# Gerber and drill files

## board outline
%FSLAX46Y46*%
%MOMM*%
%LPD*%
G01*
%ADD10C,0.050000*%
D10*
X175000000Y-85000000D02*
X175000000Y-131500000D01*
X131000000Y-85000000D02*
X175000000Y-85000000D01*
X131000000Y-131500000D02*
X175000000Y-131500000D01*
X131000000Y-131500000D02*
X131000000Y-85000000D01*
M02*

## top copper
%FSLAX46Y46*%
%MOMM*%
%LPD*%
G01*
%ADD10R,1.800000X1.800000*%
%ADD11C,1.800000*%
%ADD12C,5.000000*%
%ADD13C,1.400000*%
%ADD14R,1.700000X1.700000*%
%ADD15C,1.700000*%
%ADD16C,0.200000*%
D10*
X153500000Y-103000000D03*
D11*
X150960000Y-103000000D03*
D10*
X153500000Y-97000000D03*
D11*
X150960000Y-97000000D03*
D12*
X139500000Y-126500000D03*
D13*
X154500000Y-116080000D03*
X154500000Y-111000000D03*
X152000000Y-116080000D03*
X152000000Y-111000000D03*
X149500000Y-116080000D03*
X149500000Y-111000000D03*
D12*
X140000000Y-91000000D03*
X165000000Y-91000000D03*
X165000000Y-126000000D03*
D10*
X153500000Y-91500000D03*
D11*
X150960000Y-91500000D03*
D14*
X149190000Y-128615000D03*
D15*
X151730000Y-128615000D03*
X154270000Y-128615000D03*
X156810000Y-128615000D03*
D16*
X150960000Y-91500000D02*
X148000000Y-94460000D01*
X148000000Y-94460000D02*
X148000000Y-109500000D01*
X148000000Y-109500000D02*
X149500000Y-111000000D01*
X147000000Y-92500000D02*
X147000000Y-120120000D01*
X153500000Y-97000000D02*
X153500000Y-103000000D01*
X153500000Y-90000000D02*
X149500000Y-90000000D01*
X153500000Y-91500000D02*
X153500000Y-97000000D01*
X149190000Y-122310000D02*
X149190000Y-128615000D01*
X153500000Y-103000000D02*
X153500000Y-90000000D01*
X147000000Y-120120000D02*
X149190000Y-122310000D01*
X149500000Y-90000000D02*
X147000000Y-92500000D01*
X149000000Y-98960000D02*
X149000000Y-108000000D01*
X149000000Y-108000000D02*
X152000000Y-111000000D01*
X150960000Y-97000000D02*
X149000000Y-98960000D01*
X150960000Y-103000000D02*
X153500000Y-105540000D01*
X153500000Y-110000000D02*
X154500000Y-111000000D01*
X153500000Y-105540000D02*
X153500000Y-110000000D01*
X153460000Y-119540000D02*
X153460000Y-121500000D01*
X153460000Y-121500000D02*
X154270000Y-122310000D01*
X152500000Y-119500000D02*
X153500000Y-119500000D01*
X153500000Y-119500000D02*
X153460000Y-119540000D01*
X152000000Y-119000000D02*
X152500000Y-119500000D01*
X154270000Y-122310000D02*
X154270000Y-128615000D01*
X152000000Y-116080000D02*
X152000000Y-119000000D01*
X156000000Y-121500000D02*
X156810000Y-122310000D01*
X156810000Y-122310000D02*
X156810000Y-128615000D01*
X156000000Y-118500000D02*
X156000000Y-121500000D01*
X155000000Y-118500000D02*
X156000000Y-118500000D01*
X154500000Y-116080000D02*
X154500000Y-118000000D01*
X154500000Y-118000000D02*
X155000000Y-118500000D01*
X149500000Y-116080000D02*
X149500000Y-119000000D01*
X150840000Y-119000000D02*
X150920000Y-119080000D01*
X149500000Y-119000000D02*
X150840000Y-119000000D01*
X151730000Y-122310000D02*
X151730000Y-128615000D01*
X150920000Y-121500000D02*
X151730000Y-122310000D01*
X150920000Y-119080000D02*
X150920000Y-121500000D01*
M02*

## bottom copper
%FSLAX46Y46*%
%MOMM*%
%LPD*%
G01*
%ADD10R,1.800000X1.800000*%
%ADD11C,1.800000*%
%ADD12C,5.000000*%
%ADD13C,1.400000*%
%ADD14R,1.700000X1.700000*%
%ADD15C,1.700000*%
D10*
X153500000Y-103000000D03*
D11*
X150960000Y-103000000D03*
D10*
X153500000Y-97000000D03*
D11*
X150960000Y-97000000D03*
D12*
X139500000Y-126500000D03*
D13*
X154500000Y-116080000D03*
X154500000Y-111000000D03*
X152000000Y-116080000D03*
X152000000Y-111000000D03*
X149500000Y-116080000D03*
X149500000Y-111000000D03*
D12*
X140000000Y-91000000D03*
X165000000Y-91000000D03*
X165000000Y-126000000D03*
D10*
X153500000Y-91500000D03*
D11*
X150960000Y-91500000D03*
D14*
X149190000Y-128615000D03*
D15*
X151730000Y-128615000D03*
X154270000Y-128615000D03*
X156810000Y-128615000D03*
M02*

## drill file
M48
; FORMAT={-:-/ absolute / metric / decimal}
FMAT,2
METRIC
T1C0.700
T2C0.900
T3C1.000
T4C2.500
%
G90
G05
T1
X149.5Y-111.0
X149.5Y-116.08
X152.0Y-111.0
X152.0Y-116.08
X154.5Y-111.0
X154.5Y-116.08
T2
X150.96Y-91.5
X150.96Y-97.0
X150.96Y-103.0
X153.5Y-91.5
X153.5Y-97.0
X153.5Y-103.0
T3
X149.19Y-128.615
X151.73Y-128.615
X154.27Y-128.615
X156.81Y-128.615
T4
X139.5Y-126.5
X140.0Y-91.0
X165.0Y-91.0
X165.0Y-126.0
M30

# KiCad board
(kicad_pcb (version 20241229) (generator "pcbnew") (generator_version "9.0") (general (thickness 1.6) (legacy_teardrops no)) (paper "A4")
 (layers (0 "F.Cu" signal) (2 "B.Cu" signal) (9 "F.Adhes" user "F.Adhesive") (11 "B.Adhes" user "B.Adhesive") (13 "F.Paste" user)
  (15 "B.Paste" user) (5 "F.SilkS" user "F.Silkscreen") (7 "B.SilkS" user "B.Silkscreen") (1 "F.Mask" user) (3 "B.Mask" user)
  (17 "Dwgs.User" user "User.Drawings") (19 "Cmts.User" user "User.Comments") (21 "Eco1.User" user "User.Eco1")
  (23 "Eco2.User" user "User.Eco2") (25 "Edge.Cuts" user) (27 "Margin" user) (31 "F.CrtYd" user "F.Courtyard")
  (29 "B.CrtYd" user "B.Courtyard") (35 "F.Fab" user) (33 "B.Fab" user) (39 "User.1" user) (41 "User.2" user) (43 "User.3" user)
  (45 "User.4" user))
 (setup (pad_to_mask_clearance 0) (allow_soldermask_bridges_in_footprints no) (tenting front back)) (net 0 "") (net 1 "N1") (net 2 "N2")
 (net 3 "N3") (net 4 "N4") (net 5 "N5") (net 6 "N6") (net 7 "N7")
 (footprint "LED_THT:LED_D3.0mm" (layer "F.Cu") (at 153.5 103 180)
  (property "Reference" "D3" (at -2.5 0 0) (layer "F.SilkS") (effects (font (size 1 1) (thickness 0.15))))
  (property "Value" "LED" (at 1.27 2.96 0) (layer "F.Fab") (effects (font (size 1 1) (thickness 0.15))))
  (pad "1" thru_hole rect (at 0 0 180) (size 1.8 1.8) (drill 0.9) (layers "*.Cu" "*.Mask") (remove_unused_layers no) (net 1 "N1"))
  (pad "2" thru_hole circle (at 2.54 0 180) (size 1.8 1.8) (drill 0.9) (layers "*.Cu" "*.Mask") (remove_unused_layers no) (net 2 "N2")))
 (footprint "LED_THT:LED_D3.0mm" (layer "F.Cu") (at 153.5 97 180)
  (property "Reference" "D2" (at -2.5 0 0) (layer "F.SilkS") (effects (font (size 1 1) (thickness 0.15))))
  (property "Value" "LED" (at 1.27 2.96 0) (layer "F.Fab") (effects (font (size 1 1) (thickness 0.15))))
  (pad "1" thru_hole rect (at 0 0 180) (size 1.8 1.8) (drill 0.9) (layers "*.Cu" "*.Mask") (remove_unused_layers no) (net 1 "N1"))
  (pad "2" thru_hole circle (at 2.54 0 180) (size 1.8 1.8) (drill 0.9) (layers "*.Cu" "*.Mask") (remove_unused_layers no) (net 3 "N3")))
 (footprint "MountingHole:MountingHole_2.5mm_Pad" (layer "F.Cu") (at 139.5 126.5)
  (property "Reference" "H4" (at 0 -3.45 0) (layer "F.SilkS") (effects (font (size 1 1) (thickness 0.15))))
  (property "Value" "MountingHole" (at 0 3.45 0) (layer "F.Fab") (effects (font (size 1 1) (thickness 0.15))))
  (pad "1" thru_hole circle (at 0 0) (size 5 5) (drill 2.5) (layers "*.Cu" "*.Mask") (remove_unused_layers no) (zone_connect 2)))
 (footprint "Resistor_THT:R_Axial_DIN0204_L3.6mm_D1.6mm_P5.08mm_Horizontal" (layer "F.Cu") (at 154.5 116.08 90)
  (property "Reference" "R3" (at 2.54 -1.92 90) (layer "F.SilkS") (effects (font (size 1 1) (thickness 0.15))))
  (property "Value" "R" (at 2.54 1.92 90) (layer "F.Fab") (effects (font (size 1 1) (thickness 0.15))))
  (pad "1" thru_hole circle (at 0 0 90) (size 1.4 1.4) (drill 0.7) (layers "*.Cu" "*.Mask") (remove_unused_layers no) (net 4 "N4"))
  (pad "2" thru_hole circle (at 5.08 0 90) (size 1.4 1.4) (drill 0.7) (layers "*.Cu" "*.Mask") (remove_unused_layers no) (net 2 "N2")))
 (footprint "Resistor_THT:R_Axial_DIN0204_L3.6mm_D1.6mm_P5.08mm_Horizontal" (layer "F.Cu") (at 152 116.08 90)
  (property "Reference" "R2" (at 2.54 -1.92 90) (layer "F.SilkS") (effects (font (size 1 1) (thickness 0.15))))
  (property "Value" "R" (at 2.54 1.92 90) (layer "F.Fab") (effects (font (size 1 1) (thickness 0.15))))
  (pad "1" thru_hole circle (at 0 0 90) (size 1.4 1.4) (drill 0.7) (layers "*.Cu" "*.Mask") (remove_unused_layers no) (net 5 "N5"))
  (pad "2" thru_hole circle (at 5.08 0 90) (size 1.4 1.4) (drill 0.7) (layers "*.Cu" "*.Mask") (remove_unused_layers no) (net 3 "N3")))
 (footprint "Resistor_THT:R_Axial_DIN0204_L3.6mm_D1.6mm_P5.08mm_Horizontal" (layer "F.Cu") (at 149.5 116.08 90)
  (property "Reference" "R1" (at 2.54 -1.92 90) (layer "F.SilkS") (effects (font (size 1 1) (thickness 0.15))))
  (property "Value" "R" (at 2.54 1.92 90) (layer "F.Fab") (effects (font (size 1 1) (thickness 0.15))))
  (pad "1" thru_hole circle (at 0 0 90) (size 1.4 1.4) (drill 0.7) (layers "*.Cu" "*.Mask") (remove_unused_layers no) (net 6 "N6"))
  (pad "2" thru_hole circle (at 5.08 0 90) (size 1.4 1.4) (drill 0.7) (layers "*.Cu" "*.Mask") (remove_unused_layers no) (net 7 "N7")))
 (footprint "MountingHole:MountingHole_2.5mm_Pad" (layer "F.Cu") (at 140 91)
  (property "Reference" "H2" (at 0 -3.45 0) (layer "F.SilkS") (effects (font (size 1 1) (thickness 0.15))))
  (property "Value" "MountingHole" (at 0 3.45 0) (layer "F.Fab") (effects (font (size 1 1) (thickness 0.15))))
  (pad "1" thru_hole circle (at 0 0) (size 5 5) (drill 2.5) (layers "*.Cu" "*.Mask") (remove_unused_layers no) (zone_connect 2)))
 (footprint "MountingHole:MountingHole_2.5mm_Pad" (layer "F.Cu") (at 165 91)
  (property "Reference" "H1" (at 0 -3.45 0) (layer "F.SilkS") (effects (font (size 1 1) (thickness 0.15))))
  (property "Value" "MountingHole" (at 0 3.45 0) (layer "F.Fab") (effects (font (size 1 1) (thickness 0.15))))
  (pad "1" thru_hole circle (at 0 0) (size 5 5) (drill 2.5) (layers "*.Cu" "*.Mask") (remove_unused_layers no) (zone_connect 2)))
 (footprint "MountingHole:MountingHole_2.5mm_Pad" (layer "F.Cu") (at 165 126)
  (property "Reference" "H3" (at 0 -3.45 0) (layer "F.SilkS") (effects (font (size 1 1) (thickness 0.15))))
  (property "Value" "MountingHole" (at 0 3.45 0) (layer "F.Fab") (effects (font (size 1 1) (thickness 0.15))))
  (pad "1" thru_hole circle (at 0 0) (size 5 5) (drill 2.5) (layers "*.Cu" "*.Mask") (remove_unused_layers no) (zone_connect 2)))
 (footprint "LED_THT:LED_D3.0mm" (layer "F.Cu") (at 153.5 91.5 180)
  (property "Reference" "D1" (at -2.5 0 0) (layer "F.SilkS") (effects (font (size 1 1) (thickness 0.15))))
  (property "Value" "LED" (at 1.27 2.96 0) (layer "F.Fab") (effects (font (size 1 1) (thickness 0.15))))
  (pad "1" thru_hole rect (at 0 0 180) (size 1.8 1.8) (drill 0.9) (layers "*.Cu" "*.Mask") (remove_unused_layers no) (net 1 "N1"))
  (pad "2" thru_hole circle (at 2.54 0 180) (size 1.8 1.8) (drill 0.9) (layers "*.Cu" "*.Mask") (remove_unused_layers no) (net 7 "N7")))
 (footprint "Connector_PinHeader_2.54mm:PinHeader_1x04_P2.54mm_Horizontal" (layer "B.Cu") (at 149.19 128.615 -90)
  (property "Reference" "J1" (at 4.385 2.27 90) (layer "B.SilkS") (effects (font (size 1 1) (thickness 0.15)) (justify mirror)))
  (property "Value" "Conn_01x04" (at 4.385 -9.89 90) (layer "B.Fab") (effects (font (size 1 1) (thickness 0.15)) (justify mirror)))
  (pad "1" thru_hole rect (at 0 0 270) (size 1.7 1.7) (drill 1) (layers "*.Cu" "*.Mask") (remove_unused_layers no) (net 1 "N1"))
  (pad "2" thru_hole circle (at 0 -2.54 270) (size 1.7 1.7) (drill 1) (layers "*.Cu" "*.Mask") (remove_unused_layers no) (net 6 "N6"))
  (pad "3" thru_hole circle (at 0 -5.08 270) (size 1.7 1.7) (drill 1) (layers "*.Cu" "*.Mask") (remove_unused_layers no) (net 5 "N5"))
  (pad "4" thru_hole circle (at 0 -7.62 270) (size 1.7 1.7) (drill 1) (layers "*.Cu" "*.Mask") (remove_unused_layers no) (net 4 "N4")))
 (gr_line (start 175 85) (end 175 131.5) (stroke (width 0.05) (type default)) (layer "Edge.Cuts"))
 (gr_line (start 131 85) (end 175 85) (stroke (width 0.05) (type default)) (layer "Edge.Cuts"))
 (gr_line (start 131 131.5) (end 175 131.5) (stroke (width 0.05) (type default)) (layer "Edge.Cuts"))
 (gr_line (start 131 131.5) (end 131 85) (stroke (width 0.05) (type default)) (layer "Edge.Cuts"))
 (segment (start 150.96 91.5) (end 148 94.46) (width 0.2) (layer "F.Cu") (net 7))
 (segment (start 148 94.46) (end 148 109.5) (width 0.2) (layer "F.Cu") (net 7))
 (segment (start 148 109.5) (end 149.5 111) (width 0.2) (layer "F.Cu") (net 7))
 (segment (start 147 92.5) (end 147 120.12) (width 0.2) (layer "F.Cu") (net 1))
 (segment (start 153.5 97) (end 153.5 103) (width 0.2) (layer "F.Cu") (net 1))
 (segment (start 153.5 90) (end 149.5 90) (width 0.2) (layer "F.Cu") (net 1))
 (segment (start 153.5 91.5) (end 153.5 97) (width 0.2) (layer "F.Cu") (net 1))
 (segment (start 149.19 122.31) (end 149.19 128.615) (width 0.2) (layer "F.Cu") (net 1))
 (segment (start 153.5 103) (end 153.5 90) (width 0.2) (layer "F.Cu") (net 1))
 (segment (start 147 120.12) (end 149.19 122.31) (width 0.2) (layer "F.Cu") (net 1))
 (segment (start 149.5 90) (end 147 92.5) (width 0.2) (layer "F.Cu") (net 1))
 (segment (start 149 98.96) (end 149 108) (width 0.2) (layer "F.Cu") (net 3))
 (segment (start 149 108) (end 152 111) (width 0.2) (layer "F.Cu") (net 3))
 (segment (start 150.96 97) (end 149 98.96) (width 0.2) (layer "F.Cu") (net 3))
 (segment (start 150.96 103) (end 153.5 105.54) (width 0.2) (layer "F.Cu") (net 2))
 (segment (start 153.5 110) (end 154.5 111) (width 0.2) (layer "F.Cu") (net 2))
 (segment (start 153.5 105.54) (end 153.5 110) (width 0.2) (layer "F.Cu") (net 2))
 (segment (start 153.46 119.54) (end 153.46 121.5) (width 0.2) (layer "F.Cu") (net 5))
 (segment (start 153.46 121.5) (end 154.27 122.31) (width 0.2) (layer "F.Cu") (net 5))
 (segment (start 152.5 119.5) (end 153.5 119.5) (width 0.2) (layer "F.Cu") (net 5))
 (segment (start 153.5 119.5) (end 153.46 119.54) (width 0.2) (layer "F.Cu") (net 5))
 (segment (start 152 119) (end 152.5 119.5) (width 0.2) (layer "F.Cu") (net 5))
 (segment (start 154.27 122.31) (end 154.27 128.615) (width 0.2) (layer "F.Cu") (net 5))
 (segment (start 152 116.08) (end 152 119) (width 0.2) (layer "F.Cu") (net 5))
 (segment (start 156 121.5) (end 156.81 122.31) (width 0.2) (layer "F.Cu") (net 4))
 (segment (start 156.81 122.31) (end 156.81 128.615) (width 0.2) (layer "F.Cu") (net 4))
 (segment (start 156 118.5) (end 156 121.5) (width 0.2) (layer "F.Cu") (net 4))
 (segment (start 155 118.5) (end 156 118.5) (width 0.2) (layer "F.Cu") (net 4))
 (segment (start 154.5 116.08) (end 154.5 118) (width 0.2) (layer "F.Cu") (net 4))
 (segment (start 154.5 118) (end 155 118.5) (width 0.2) (layer "F.Cu") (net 4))
 (segment (start 149.5 116.08) (end 149.5 119) (width 0.2) (layer "F.Cu") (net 6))
 (segment (start 150.84 119) (end 150.92 119.08) (width 0.2) (layer "F.Cu") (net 6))
 (segment (start 149.5 119) (end 150.84 119) (width 0.2) (layer "F.Cu") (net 6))
 (segment (start 151.73 122.31) (end 151.73 128.615) (width 0.2) (layer "F.Cu") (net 6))
 (segment (start 150.92 121.5) (end 151.73 122.31) (width 0.2) (layer "F.Cu") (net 6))
 (segment (start 150.92 119.08) (end 150.92 121.5) (width 0.2) (layer "F.Cu") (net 6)))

